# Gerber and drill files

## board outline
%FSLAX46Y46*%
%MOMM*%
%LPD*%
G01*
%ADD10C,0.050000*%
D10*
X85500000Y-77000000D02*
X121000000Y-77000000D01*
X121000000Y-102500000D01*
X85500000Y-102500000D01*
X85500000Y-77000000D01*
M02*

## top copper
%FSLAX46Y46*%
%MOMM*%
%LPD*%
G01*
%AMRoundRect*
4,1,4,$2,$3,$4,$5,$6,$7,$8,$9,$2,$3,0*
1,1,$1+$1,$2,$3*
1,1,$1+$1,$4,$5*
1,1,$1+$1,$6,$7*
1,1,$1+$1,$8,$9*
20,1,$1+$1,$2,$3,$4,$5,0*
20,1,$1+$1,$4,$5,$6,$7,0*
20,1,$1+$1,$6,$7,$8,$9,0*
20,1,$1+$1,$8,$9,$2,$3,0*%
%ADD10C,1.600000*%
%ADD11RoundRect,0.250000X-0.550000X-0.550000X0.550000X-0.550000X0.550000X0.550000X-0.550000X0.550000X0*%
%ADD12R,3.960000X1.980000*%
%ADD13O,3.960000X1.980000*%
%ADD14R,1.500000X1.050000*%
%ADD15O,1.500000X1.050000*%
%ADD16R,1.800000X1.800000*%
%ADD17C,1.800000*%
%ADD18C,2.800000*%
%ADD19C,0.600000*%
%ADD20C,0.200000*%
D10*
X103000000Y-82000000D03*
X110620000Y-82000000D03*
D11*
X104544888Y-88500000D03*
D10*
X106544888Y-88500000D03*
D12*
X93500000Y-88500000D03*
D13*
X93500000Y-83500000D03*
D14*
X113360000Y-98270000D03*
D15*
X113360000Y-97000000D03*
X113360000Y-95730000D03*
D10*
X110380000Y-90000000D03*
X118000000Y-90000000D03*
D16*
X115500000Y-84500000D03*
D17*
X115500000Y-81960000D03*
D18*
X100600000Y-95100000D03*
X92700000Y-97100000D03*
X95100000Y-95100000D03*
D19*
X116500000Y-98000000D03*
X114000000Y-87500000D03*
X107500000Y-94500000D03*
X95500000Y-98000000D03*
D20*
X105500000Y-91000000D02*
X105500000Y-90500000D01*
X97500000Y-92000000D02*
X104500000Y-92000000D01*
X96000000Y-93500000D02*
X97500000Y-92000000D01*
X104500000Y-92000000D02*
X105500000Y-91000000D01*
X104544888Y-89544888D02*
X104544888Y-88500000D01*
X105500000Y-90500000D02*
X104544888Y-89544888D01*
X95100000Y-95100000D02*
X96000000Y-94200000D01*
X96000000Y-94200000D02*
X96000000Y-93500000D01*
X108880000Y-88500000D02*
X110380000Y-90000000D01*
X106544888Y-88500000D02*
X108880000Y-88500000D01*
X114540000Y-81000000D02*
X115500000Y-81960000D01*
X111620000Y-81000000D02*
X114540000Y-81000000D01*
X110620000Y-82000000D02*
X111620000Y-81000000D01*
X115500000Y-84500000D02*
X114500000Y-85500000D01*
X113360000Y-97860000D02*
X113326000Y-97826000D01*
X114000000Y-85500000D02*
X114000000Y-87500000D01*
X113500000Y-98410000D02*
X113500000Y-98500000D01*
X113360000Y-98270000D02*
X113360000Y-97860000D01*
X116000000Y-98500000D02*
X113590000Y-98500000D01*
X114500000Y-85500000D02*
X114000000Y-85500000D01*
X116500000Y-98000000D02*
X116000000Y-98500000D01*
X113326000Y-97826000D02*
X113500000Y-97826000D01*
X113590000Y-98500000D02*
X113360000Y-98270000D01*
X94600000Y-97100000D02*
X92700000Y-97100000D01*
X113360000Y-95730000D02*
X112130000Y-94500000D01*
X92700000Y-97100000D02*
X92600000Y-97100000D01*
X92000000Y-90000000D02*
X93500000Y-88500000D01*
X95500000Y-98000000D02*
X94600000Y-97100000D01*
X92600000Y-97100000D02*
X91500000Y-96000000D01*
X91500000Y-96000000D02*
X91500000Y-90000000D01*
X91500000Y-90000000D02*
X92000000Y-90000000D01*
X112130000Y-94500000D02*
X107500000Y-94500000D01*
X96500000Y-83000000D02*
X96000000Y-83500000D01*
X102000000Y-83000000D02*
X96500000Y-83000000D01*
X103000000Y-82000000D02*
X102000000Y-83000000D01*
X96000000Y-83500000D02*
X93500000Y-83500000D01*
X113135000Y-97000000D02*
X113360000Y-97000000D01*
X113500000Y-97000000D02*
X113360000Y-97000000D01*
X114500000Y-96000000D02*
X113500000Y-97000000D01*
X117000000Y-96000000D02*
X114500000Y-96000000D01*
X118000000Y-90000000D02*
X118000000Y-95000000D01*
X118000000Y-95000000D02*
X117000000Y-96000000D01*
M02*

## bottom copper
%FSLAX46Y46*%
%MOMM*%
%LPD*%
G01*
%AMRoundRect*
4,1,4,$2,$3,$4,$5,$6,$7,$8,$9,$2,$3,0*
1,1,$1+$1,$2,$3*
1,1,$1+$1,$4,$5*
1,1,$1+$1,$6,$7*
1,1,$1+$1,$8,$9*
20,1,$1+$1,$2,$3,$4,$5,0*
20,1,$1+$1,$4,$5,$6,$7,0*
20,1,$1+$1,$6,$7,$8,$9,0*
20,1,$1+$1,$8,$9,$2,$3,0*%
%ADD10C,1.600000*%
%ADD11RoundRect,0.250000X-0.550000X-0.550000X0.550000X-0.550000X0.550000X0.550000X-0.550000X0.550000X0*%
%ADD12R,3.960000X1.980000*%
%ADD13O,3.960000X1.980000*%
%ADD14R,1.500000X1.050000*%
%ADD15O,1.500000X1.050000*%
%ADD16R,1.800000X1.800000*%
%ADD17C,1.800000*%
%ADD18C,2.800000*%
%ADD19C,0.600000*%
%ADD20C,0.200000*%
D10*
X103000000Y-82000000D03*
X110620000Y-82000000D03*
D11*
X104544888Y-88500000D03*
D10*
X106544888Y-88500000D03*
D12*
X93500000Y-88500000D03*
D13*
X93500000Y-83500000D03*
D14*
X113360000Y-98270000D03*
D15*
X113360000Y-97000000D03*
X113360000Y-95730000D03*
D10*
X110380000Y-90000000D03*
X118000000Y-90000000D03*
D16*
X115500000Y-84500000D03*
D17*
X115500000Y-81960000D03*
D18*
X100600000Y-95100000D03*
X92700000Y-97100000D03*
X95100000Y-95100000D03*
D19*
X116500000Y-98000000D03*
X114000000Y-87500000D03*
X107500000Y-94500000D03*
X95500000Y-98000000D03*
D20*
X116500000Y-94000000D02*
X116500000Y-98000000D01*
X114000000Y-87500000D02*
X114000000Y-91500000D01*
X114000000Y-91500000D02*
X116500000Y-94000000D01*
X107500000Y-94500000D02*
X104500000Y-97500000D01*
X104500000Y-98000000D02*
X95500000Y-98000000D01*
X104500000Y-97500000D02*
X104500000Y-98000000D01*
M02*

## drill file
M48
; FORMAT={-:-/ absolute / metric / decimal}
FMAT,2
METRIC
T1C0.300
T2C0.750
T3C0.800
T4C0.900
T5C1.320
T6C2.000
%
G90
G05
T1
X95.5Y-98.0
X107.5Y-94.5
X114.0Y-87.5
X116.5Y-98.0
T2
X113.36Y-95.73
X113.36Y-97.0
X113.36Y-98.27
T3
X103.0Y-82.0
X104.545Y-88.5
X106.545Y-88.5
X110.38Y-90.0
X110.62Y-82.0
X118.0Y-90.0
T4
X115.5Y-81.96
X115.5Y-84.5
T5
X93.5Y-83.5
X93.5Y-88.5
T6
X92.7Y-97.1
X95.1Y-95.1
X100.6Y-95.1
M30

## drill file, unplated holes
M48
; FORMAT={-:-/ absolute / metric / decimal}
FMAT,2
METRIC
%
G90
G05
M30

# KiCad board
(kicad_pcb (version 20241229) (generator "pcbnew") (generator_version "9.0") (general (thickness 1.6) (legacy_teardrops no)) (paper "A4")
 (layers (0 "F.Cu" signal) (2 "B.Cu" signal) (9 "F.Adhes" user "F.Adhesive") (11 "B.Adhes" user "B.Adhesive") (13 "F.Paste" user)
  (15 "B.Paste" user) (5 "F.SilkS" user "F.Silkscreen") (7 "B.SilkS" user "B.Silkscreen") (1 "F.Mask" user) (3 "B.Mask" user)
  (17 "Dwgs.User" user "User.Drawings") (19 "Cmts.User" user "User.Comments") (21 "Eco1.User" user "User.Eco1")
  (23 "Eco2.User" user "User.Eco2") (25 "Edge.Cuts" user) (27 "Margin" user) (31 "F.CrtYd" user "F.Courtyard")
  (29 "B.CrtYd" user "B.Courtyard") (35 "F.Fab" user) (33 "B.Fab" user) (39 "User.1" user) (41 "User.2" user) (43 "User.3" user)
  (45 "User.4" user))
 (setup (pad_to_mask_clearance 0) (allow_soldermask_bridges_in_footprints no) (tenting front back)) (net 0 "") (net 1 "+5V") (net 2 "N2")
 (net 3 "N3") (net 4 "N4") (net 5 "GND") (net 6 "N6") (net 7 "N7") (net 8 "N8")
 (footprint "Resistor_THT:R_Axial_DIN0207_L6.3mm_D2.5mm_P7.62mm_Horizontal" (layer "F.Cu") (at 103 82)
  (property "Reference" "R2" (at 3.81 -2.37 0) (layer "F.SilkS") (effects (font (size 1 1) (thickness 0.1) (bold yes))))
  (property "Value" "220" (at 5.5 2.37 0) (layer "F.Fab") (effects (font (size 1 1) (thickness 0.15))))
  (pad "1" thru_hole circle (at 0 0) (size 1.6 1.6) (drill 0.8) (layers "*.Cu" "*.Mask") (remove_unused_layers no) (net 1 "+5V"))
  (pad "2" thru_hole circle (at 7.62 0) (size 1.6 1.6) (drill 0.8) (layers "*.Cu" "*.Mask") (remove_unused_layers no) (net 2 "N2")))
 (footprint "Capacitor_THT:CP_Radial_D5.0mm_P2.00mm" (layer "F.Cu") (at 104.544888 88.5)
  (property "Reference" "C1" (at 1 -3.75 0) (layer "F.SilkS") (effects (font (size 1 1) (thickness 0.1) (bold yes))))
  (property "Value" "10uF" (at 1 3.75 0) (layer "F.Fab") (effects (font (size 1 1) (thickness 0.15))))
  (pad "1" thru_hole roundrect (at 0 0) (size 1.6 1.6) (drill 0.8) (layers "*.Cu" "*.Mask") (remove_unused_layers no)
   (roundrect_rratio 0.15625) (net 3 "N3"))
  (pad "2" thru_hole circle (at 2 0) (size 1.6 1.6) (drill 0.8) (layers "*.Cu" "*.Mask") (remove_unused_layers no) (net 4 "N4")))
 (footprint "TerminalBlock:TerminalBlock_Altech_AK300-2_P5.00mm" (layer "F.Cu") (at 93.5 88.5 90)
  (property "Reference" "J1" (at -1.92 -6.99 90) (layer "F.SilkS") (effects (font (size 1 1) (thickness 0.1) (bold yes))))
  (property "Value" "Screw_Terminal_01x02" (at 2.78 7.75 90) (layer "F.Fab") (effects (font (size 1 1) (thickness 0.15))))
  (pad "1" thru_hole rect (at 0 0 90) (size 1.98 3.96) (drill 1.32) (layers "*.Cu" "*.Mask") (remove_unused_layers no) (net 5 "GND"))
  (pad "2" thru_hole oval (at 5 0 90) (size 1.98 3.96) (drill 1.32) (layers "*.Cu" "*.Mask") (remove_unused_layers no) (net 1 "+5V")))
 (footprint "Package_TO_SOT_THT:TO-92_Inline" (layer "F.Cu") (at 113.36 98.27 90)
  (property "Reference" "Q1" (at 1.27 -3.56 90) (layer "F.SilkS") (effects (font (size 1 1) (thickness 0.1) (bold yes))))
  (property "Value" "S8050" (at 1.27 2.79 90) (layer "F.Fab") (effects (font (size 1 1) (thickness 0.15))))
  (pad "1" thru_hole rect (at 0 0 90) (size 1.05 1.5) (drill 0.75) (layers "*.Cu" "*.Mask") (remove_unused_layers no) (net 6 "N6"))
  (pad "2" thru_hole oval (at 1.27 0 90) (size 1.05 1.5) (drill 0.75) (layers "*.Cu" "*.Mask") (remove_unused_layers no) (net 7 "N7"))
  (pad "3" thru_hole oval (at 2.54 0 90) (size 1.05 1.5) (drill 0.75) (layers "*.Cu" "*.Mask") (remove_unused_layers no) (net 5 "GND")))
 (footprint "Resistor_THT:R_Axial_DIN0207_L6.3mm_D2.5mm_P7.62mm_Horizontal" (layer "F.Cu") (at 110.38 90)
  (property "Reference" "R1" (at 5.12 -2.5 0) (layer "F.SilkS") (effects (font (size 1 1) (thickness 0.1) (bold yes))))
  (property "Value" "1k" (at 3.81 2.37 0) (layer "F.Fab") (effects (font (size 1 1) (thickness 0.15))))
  (pad "1" thru_hole circle (at 0 0) (size 1.6 1.6) (drill 0.8) (layers "*.Cu" "*.Mask") (remove_unused_layers no) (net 4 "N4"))
  (pad "2" thru_hole circle (at 7.62 0) (size 1.6 1.6) (drill 0.8) (layers "*.Cu" "*.Mask") (remove_unused_layers no) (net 7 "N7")))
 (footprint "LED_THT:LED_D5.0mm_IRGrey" (layer "F.Cu") (at 115.5 84.5 90)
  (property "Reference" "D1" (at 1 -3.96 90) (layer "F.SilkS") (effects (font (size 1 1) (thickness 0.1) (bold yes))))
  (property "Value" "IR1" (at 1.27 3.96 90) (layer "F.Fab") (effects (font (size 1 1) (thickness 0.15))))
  (pad "1" thru_hole rect (at 0 0 90) (size 1.8 1.8) (drill 0.9) (layers "*.Cu" "*.Mask") (remove_unused_layers no) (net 6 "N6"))
  (pad "2" thru_hole circle (at 2.54 0 90) (size 1.8 1.8) (drill 0.9) (layers "*.Cu" "*.Mask") (remove_unused_layers no) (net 2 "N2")))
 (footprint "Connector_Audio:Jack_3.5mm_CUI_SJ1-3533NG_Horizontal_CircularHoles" (layer "F.Cu") (at 92.7 97.1 90)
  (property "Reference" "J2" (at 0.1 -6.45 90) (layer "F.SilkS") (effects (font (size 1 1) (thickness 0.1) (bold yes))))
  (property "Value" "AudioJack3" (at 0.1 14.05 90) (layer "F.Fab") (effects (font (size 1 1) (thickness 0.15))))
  (pad "R" thru_hole circle (at 2 7.9 90) (size 2.8 2.8) (drill 2) (layers "*.Cu" "*.Mask") (remove_unused_layers no) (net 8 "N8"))
  (pad "S" thru_hole circle (at 0 0 90) (size 2.8 2.8) (drill 2) (layers "*.Cu" "*.Mask") (remove_unused_layers no) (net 5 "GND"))
  (pad "T" thru_hole circle (at 2 2.4 90) (size 2.8 2.8) (drill 2) (layers "*.Cu" "*.Mask") (remove_unused_layers no) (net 3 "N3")))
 (gr_rect (start 85.5 77) (end 121 102.5) (stroke (width 0.05) (type default)) (fill no) (layer "Edge.Cuts"))
 (segment (start 105.5 91) (end 105.5 90.5) (width 0.2) (layer "F.Cu") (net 3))
 (segment (start 97.5 92) (end 104.5 92) (width 0.2) (layer "F.Cu") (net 3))
 (segment (start 96 93.5) (end 97.5 92) (width 0.2) (layer "F.Cu") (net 3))
 (segment (start 104.5 92) (end 105.5 91) (width 0.2) (layer "F.Cu") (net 3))
 (segment (start 104.544888 89.544888) (end 104.544888 88.5) (width 0.2) (layer "F.Cu") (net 3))
 (segment (start 105.5 90.5) (end 104.544888 89.544888) (width 0.2) (layer "F.Cu") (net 3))
 (segment (start 95.1 95.1) (end 96 94.2) (width 0.2) (layer "F.Cu") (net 3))
 (segment (start 96 94.2) (end 96 93.5) (width 0.2) (layer "F.Cu") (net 3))
 (segment (start 108.88 88.5) (end 110.38 90) (width 0.2) (layer "F.Cu") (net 4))
 (segment (start 106.544888 88.5) (end 108.88 88.5) (width 0.2) (layer "F.Cu") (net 4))
 (segment (start 114.54 81) (end 115.5 81.96) (width 0.2) (layer "F.Cu") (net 2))
 (segment (start 111.62 81) (end 114.54 81) (width 0.2) (layer "F.Cu") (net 2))
 (segment (start 110.62 82) (end 111.62 81) (width 0.2) (layer "F.Cu") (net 2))
 (segment (start 115.5 84.5) (end 114.5 85.5) (width 0.2) (layer "F.Cu") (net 6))
 (segment (start 113.36 97.86) (end 113.326 97.826) (width 0.2) (layer "F.Cu") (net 6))
 (segment (start 114 85.5) (end 114 87.5) (width 0.2) (layer "F.Cu") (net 6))
 (segment (start 113.5 98.41) (end 113.5 98.5) (width 0.2) (layer "F.Cu") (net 6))
 (segment (start 113.36 98.27) (end 113.36 97.86) (width 0.2) (layer "F.Cu") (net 6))
 (segment (start 116 98.5) (end 113.59 98.5) (width 0.2) (layer "F.Cu") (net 6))
 (segment (start 114.5 85.5) (end 114 85.5) (width 0.2) (layer "F.Cu") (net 6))
 (segment (start 116.5 98) (end 116 98.5) (width 0.2) (layer "F.Cu") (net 6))
 (segment (start 113.326 97.826) (end 113.5 97.826) (width 0.2) (layer "F.Cu") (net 6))
 (segment (start 113.59 98.5) (end 113.36 98.27) (width 0.2) (layer "F.Cu") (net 6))
 (via (at 116.5 98) (size 0.6) (drill 0.3) (layers "F.Cu" "B.Cu") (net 6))
 (via (at 114 87.5) (size 0.6) (drill 0.3) (layers "F.Cu" "B.Cu") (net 6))
 (segment (start 116.5 94) (end 116.5 98) (width 0.2) (layer "B.Cu") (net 6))
 (segment (start 114 87.5) (end 114 91.5) (width 0.2) (layer "B.Cu") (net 6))
 (segment (start 114 91.5) (end 116.5 94) (width 0.2) (layer "B.Cu") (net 6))
 (segment (start 94.6 97.1) (end 92.7 97.1) (width 0.2) (layer "F.Cu") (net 5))
 (segment (start 113.36 95.73) (end 112.13 94.5) (width 0.2) (layer "F.Cu") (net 5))
 (segment (start 92.7 97.1) (end 92.6 97.1) (width 0.2) (layer "F.Cu") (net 5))
 (segment (start 92 90) (end 93.5 88.5) (width 0.2) (layer "F.Cu") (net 5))
 (segment (start 95.5 98) (end 94.6 97.1) (width 0.2) (layer "F.Cu") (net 5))
 (segment (start 92.6 97.1) (end 91.5 96) (width 0.2) (layer "F.Cu") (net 5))
 (segment (start 91.5 96) (end 91.5 90) (width 0.2) (layer "F.Cu") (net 5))
 (segment (start 91.5 90) (end 92 90) (width 0.2) (layer "F.Cu") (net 5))
 (segment (start 112.13 94.5) (end 107.5 94.5) (width 0.2) (layer "F.Cu") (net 5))
 (via (at 107.5 94.5) (size 0.6) (drill 0.3) (layers "F.Cu" "B.Cu") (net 5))
 (via (at 95.5 98) (size 0.6) (drill 0.3) (layers "F.Cu" "B.Cu") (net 5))
 (segment (start 107.5 94.5) (end 104.5 97.5) (width 0.2) (layer "B.Cu") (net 5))
 (segment (start 104.5 98) (end 95.5 98) (width 0.2) (layer "B.Cu") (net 5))
 (segment (start 104.5 97.5) (end 104.5 98) (width 0.2) (layer "B.Cu") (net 5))
 (segment (start 96.5 83) (end 96 83.5) (width 0.2) (layer "F.Cu") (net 1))
 (segment (start 102 83) (end 96.5 83) (width 0.2) (layer "F.Cu") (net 1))
 (segment (start 103 82) (end 102 83) (width 0.2) (layer "F.Cu") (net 1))
 (segment (start 96 83.5) (end 93.5 83.5) (width 0.2) (layer "F.Cu") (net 1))
 (segment (start 113.135 97) (end 113.36 97) (width 0.2) (layer "F.Cu") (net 7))
 (segment (start 113.5 97) (end 113.36 97) (width 0.2) (layer "F.Cu") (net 7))
 (segment (start 114.5 96) (end 113.5 97) (width 0.2) (layer "F.Cu") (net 7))
 (segment (start 117 96) (end 114.5 96) (width 0.2) (layer "F.Cu") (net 7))
 (segment (start 118 90) (end 118 95) (width 0.2) (layer "F.Cu") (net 7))
 (segment (start 118 95) (end 117 96) (width 0.2) (layer "F.Cu") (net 7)))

